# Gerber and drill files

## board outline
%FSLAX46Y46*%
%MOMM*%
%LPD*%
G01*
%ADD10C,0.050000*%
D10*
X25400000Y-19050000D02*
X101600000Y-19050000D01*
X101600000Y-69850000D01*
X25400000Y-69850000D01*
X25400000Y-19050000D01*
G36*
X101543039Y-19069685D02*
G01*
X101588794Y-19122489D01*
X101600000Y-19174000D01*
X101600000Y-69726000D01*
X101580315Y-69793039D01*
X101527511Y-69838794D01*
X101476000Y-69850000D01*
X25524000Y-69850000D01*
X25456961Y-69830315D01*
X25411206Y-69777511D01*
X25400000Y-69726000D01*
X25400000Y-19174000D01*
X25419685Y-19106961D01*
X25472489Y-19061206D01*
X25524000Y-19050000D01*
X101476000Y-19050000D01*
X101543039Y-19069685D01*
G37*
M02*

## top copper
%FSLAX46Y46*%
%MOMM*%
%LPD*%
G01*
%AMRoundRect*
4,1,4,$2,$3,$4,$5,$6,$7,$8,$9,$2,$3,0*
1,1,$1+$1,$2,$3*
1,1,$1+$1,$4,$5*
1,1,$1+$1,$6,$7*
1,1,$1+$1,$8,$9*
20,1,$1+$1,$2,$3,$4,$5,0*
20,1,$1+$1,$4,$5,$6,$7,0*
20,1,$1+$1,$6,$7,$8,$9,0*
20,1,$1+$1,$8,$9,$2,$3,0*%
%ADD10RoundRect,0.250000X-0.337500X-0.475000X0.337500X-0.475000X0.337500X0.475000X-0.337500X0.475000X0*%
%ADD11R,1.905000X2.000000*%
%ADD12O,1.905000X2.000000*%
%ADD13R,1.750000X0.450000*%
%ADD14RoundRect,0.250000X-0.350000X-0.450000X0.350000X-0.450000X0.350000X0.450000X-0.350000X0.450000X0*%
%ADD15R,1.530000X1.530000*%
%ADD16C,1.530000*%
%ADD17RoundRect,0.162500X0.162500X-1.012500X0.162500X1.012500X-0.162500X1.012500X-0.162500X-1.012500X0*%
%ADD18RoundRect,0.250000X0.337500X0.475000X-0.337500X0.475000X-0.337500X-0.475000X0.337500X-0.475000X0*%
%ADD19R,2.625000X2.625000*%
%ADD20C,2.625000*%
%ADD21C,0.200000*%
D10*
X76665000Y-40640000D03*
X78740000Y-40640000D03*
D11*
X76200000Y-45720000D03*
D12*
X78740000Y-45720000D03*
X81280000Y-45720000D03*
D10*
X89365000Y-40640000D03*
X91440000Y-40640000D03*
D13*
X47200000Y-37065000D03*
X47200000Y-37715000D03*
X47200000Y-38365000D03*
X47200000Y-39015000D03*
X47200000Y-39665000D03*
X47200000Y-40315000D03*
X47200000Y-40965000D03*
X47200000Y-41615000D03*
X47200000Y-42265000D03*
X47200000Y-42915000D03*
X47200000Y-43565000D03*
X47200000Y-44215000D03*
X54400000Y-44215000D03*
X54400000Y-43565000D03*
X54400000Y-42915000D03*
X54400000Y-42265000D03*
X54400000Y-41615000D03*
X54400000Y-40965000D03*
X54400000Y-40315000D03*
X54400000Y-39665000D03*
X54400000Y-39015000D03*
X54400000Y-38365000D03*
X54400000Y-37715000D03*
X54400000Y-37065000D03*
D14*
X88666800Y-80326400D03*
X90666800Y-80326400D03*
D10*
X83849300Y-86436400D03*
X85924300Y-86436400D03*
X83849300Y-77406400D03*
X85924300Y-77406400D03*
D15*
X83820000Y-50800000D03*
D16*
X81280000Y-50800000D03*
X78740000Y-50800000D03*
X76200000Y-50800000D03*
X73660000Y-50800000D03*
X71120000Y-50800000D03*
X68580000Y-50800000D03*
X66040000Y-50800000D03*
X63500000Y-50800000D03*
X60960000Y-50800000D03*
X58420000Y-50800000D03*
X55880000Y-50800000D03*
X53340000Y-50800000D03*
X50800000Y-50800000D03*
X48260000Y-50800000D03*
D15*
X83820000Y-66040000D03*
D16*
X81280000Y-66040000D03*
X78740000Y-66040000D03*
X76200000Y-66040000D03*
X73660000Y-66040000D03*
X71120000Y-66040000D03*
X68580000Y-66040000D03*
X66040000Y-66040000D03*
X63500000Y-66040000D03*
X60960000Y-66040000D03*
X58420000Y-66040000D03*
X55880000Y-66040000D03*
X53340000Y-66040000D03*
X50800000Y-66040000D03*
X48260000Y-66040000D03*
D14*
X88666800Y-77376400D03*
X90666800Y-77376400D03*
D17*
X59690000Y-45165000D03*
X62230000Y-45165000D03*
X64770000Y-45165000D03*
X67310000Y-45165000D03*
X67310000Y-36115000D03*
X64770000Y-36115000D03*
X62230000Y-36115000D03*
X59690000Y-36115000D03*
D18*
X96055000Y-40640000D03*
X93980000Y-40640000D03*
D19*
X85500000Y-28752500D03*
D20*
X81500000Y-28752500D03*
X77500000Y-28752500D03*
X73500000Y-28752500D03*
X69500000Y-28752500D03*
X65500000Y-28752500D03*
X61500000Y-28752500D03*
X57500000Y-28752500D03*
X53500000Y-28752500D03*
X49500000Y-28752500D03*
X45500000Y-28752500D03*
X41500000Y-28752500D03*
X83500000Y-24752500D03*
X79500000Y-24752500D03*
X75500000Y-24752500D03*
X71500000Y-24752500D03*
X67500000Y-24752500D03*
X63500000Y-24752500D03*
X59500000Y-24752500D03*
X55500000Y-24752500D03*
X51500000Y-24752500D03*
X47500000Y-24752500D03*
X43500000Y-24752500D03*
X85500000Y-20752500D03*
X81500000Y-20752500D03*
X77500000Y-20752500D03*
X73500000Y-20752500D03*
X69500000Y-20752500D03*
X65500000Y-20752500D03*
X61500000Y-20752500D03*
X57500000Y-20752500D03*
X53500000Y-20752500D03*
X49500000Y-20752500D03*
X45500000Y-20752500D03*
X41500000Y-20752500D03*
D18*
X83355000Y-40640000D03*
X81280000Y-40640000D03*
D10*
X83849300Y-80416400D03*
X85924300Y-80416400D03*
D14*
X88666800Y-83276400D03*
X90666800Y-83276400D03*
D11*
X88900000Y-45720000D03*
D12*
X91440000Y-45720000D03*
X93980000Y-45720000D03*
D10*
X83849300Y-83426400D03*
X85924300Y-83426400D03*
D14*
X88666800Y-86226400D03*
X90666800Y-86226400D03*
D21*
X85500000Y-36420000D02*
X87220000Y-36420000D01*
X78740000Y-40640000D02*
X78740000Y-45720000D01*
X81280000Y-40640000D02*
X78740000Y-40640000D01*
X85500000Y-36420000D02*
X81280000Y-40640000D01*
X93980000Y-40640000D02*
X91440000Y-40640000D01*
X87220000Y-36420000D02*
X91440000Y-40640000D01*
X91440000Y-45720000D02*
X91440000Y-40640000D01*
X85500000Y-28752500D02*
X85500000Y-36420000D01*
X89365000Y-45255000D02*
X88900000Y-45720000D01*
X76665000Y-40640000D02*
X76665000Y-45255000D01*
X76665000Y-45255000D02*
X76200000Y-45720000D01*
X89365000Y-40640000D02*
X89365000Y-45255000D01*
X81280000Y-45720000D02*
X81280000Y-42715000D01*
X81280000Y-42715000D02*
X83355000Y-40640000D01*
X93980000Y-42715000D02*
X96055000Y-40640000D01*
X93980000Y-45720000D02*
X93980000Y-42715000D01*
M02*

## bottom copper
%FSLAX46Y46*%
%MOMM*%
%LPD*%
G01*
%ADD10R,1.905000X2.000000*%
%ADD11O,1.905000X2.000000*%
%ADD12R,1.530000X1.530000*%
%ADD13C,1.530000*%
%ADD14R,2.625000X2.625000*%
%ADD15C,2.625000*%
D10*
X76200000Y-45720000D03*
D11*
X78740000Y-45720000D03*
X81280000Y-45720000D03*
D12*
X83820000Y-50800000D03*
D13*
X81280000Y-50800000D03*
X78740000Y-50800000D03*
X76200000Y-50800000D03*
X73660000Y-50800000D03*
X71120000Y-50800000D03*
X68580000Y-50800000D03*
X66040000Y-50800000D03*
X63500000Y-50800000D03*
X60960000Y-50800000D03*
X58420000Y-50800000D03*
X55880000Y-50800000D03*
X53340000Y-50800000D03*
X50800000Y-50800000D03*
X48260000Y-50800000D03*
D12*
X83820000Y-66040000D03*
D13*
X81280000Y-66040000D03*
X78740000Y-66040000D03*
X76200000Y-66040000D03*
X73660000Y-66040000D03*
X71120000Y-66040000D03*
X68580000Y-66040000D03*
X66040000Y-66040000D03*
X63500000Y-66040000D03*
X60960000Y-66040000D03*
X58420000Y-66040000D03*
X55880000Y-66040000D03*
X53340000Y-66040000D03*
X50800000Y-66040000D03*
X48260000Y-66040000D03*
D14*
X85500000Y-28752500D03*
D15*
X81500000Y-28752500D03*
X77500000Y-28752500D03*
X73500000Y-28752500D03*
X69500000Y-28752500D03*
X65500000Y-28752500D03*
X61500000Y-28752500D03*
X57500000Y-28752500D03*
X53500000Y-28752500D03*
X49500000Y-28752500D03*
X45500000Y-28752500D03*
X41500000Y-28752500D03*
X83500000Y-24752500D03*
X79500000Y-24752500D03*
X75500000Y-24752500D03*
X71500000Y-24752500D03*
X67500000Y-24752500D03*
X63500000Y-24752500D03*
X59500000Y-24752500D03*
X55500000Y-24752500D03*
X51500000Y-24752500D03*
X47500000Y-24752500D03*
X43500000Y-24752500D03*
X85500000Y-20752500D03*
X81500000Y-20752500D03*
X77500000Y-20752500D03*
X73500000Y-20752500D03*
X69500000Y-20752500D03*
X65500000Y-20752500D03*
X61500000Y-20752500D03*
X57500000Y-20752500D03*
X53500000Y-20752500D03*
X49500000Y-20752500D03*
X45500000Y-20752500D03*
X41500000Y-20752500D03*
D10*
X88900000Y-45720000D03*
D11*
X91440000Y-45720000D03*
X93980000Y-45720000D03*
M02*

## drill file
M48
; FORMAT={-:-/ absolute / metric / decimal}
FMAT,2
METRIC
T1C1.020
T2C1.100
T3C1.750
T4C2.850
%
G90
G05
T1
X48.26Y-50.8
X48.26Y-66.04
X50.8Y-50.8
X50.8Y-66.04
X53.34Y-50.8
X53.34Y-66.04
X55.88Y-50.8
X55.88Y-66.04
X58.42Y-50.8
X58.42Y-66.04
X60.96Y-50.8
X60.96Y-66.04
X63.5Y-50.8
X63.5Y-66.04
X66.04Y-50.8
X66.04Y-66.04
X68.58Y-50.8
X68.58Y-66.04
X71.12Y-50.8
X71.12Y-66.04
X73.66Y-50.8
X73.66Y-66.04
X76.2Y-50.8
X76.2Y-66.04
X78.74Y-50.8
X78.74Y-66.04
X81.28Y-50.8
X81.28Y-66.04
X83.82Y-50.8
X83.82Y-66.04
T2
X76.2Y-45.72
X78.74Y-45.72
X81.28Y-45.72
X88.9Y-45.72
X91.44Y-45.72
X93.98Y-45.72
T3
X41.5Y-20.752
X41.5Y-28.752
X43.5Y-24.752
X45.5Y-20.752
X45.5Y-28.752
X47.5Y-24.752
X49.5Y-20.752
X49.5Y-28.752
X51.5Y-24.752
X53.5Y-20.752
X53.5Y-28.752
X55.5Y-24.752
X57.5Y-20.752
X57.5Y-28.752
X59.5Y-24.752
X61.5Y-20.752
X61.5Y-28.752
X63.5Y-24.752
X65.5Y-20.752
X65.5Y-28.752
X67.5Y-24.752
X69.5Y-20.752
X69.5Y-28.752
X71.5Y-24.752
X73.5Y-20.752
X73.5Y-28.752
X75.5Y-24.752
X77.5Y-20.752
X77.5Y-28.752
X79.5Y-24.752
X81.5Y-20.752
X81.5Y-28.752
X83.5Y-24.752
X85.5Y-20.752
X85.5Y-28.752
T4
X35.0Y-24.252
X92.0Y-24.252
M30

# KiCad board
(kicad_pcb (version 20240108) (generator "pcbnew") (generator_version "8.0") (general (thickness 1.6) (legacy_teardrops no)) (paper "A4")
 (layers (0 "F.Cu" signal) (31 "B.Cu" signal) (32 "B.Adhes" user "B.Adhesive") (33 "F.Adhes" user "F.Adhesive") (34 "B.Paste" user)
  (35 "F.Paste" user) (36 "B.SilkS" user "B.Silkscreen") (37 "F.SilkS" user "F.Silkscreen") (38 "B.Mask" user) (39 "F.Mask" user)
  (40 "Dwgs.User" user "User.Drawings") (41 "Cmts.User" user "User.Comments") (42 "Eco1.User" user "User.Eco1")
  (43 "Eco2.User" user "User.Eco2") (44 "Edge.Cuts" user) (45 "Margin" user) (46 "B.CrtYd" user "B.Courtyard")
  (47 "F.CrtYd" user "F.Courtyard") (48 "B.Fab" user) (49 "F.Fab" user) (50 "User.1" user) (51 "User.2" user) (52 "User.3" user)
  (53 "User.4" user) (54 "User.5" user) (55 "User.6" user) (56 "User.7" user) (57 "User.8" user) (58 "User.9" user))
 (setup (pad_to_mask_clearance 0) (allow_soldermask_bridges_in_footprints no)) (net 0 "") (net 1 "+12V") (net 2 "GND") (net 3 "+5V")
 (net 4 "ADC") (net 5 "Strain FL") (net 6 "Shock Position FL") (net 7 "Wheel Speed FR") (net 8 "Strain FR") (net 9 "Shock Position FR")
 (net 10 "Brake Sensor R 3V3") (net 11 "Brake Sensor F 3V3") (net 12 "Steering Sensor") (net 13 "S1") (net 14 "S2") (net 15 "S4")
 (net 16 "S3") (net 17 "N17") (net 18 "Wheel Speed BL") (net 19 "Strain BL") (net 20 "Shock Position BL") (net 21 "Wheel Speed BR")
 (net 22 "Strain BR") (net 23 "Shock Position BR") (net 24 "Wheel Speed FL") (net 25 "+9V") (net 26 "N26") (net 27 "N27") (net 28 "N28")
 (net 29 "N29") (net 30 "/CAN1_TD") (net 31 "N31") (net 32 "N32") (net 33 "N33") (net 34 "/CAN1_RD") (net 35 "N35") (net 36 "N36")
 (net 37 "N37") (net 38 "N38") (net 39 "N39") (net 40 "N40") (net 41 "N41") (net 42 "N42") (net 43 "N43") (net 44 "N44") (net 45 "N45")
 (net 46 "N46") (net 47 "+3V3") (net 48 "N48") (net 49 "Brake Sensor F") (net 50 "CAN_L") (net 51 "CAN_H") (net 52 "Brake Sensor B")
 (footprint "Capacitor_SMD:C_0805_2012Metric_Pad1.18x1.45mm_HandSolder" (layer "F.Cu") (at 77.7025 40.64)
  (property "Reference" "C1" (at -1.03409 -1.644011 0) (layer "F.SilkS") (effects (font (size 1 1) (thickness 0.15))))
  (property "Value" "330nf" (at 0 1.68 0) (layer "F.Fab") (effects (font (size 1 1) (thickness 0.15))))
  (pad "1" smd roundrect (at -1.0375 0) (size 1.175 1.45) (layers "F.Cu" "F.Paste" "F.Mask") (roundrect_rratio 0.212766) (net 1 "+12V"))
  (pad "2" smd roundrect (at 1.0375 0) (size 1.175 1.45) (layers "F.Cu" "F.Paste" "F.Mask") (roundrect_rratio 0.212766) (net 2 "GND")))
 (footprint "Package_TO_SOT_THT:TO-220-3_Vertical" (layer "F.Cu") (at 76.2 45.72)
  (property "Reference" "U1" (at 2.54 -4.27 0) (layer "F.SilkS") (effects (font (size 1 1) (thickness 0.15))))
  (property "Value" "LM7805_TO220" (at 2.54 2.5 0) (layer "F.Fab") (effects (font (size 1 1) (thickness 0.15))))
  (pad "1" thru_hole rect (at 0 0) (size 1.905 2) (drill 1.1) (layers "*.Cu" "*.Mask") (remove_unused_layers no) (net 1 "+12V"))
  (pad "2" thru_hole oval (at 2.54 0) (size 1.905 2) (drill 1.1) (layers "*.Cu" "*.Mask") (remove_unused_layers no) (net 2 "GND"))
  (pad "3" thru_hole oval (at 5.08 0) (size 1.905 2) (drill 1.1) (layers "*.Cu" "*.Mask") (remove_unused_layers no) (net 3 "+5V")))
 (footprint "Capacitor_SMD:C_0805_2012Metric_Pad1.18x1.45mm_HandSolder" (layer "F.Cu") (at 90.4025 40.64)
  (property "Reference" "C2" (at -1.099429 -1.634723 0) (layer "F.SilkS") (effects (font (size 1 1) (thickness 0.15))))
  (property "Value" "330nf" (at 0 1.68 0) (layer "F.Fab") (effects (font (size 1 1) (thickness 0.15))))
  (pad "1" smd roundrect (at -1.0375 0) (size 1.175 1.45) (layers "F.Cu" "F.Paste" "F.Mask") (roundrect_rratio 0.212766) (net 1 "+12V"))
  (pad "2" smd roundrect (at 1.0375 0) (size 1.175 1.45) (layers "F.Cu" "F.Paste" "F.Mask") (roundrect_rratio 0.212766) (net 2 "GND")))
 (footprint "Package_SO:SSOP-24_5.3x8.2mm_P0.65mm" (layer "F.Cu") (at 50.8 40.64)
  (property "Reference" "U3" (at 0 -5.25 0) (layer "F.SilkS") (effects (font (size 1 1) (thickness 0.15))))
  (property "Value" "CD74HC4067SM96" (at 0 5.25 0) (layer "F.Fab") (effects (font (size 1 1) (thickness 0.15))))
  (pad "1" smd rect (at -3.6 -3.575) (size 1.75 0.45) (layers "F.Cu" "F.Paste" "F.Mask") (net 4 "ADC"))
  (pad "2" smd rect (at -3.6 -2.925) (size 1.75 0.45) (layers "F.Cu" "F.Paste" "F.Mask") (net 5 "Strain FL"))
  (pad "3" smd rect (at -3.6 -2.275) (size 1.75 0.45) (layers "F.Cu" "F.Paste" "F.Mask") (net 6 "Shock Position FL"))
  (pad "4" smd rect (at -3.6 -1.625) (size 1.75 0.45) (layers "F.Cu" "F.Paste" "F.Mask") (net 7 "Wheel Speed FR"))
  (pad "5" smd rect (at -3.6 -0.975) (size 1.75 0.45) (layers "F.Cu" "F.Paste" "F.Mask") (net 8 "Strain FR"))
  (pad "6" smd rect (at -3.6 -0.325) (size 1.75 0.45) (layers "F.Cu" "F.Paste" "F.Mask") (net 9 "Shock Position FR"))
  (pad "7" smd rect (at -3.6 0.325) (size 1.75 0.45) (layers "F.Cu" "F.Paste" "F.Mask") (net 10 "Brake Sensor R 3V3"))
  (pad "8" smd rect (at -3.6 0.975) (size 1.75 0.45) (layers "F.Cu" "F.Paste" "F.Mask") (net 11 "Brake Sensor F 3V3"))
  (pad "9" smd rect (at -3.6 1.625) (size 1.75 0.45) (layers "F.Cu" "F.Paste" "F.Mask") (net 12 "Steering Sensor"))
  (pad "10" smd rect (at -3.6 2.275) (size 1.75 0.45) (layers "F.Cu" "F.Paste" "F.Mask") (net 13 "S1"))
  (pad "11" smd rect (at -3.6 2.925) (size 1.75 0.45) (layers "F.Cu" "F.Paste" "F.Mask") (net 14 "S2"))
  (pad "12" smd rect (at -3.6 3.575) (size 1.75 0.45) (layers "F.Cu" "F.Paste" "F.Mask") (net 2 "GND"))
  (pad "13" smd rect (at 3.6 3.575) (size 1.75 0.45) (layers "F.Cu" "F.Paste" "F.Mask") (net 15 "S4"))
  (pad "14" smd rect (at 3.6 2.925) (size 1.75 0.45) (layers "F.Cu" "F.Paste" "F.Mask") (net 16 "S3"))
  (pad "15" smd rect (at 3.6 2.275) (size 1.75 0.45) (layers "F.Cu" "F.Paste" "F.Mask") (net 2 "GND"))
  (pad "16" smd rect (at 3.6 1.625) (size 1.75 0.45) (layers "F.Cu" "F.Paste" "F.Mask") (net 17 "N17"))
  (pad "17" smd rect (at 3.6 0.975) (size 1.75 0.45) (layers "F.Cu" "F.Paste" "F.Mask") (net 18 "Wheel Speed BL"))
  (pad "18" smd rect (at 3.6 0.325) (size 1.75 0.45) (layers "F.Cu" "F.Paste" "F.Mask") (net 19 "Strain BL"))
  (pad "19" smd rect (at 3.6 -0.325) (size 1.75 0.45) (layers "F.Cu" "F.Paste" "F.Mask") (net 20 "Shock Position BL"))
  (pad "20" smd rect (at 3.6 -0.975) (size 1.75 0.45) (layers "F.Cu" "F.Paste" "F.Mask") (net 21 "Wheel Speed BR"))
  (pad "21" smd rect (at 3.6 -1.625) (size 1.75 0.45) (layers "F.Cu" "F.Paste" "F.Mask") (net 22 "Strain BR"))
  (pad "22" smd rect (at 3.6 -2.275) (size 1.75 0.45) (layers "F.Cu" "F.Paste" "F.Mask") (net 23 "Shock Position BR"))
  (pad "23" smd rect (at 3.6 -2.925) (size 1.75 0.45) (layers "F.Cu" "F.Paste" "F.Mask") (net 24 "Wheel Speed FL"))
  (pad "24" smd rect (at 3.6 -3.575) (size 1.75 0.45) (layers "F.Cu" "F.Paste" "F.Mask") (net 3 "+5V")))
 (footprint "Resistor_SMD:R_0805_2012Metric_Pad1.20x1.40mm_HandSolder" (layer "F.Cu") (at 89.6668 80.3264)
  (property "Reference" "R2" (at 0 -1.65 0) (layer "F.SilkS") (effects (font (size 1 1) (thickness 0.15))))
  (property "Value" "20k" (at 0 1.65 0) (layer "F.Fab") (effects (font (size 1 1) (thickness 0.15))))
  (pad "1" smd roundrect (at -1 0) (size 1.2 1.4) (layers "F.Cu" "F.Paste" "F.Mask") (roundrect_rratio 0.208333) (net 2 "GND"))
  (pad "2" smd roundrect (at 1 0) (size 1.2 1.4) (layers "F.Cu" "F.Paste" "F.Mask") (roundrect_rratio 0.208333)
   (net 11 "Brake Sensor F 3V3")))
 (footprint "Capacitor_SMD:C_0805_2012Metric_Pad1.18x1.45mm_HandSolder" (layer "F.Cu") (at 84.8868 86.4364)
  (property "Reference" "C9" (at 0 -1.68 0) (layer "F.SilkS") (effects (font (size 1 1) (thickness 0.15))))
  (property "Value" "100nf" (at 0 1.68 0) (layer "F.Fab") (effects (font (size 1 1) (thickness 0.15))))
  (pad "1" smd roundrect (at -1.0375 0) (size 1.175 1.45) (layers "F.Cu" "F.Paste" "F.Mask") (roundrect_rratio 0.212766) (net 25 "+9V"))
  (pad "2" smd roundrect (at 1.0375 0) (size 1.175 1.45) (layers "F.Cu" "F.Paste" "F.Mask") (roundrect_rratio 0.212766) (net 2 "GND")))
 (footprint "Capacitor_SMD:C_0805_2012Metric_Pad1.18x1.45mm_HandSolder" (layer "F.Cu") (at 84.8868 77.4064)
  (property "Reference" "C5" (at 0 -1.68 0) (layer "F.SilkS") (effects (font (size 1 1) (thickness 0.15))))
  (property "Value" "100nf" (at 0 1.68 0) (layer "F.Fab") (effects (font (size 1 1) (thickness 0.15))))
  (pad "1" smd roundrect (at -1.0375 0) (size 1.175 1.45) (layers "F.Cu" "F.Paste" "F.Mask") (roundrect_rratio 0.212766) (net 3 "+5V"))
  (pad "2" smd roundrect (at 1.0375 0) (size 1.175 1.45) (layers "F.Cu" "F.Paste" "F.Mask") (roundrect_rratio 0.212766) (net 2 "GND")))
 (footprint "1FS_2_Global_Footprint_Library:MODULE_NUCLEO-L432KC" (layer "F.Cu") (at 67.605 58.42 -90)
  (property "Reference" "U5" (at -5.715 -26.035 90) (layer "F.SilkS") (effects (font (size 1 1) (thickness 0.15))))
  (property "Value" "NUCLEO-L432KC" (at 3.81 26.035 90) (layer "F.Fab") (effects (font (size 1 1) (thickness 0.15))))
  (pad "CN3_1" thru_hole rect (at -7.62 -16.215 270) (size 1.53 1.53) (drill 1.02) (layers "*.Cu" "*.Mask") (remove_unused_layers no)
   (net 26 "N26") (solder_mask_margin 0.102))
  (pad "CN3_2" thru_hole circle (at -7.62 -13.675 270) (size 1.53 1.53) (drill 1.02) (layers "*.Cu" "*.Mask") (remove_unused_layers no)
   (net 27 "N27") (solder_mask_margin 0.102))
  (pad "CN3_3" thru_hole circle (at -7.62 -11.135 270) (size 1.53 1.53) (drill 1.02) (layers "*.Cu" "*.Mask") (remove_unused_layers no)
   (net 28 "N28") (solder_mask_margin 0.102))
  (pad "CN3_4" thru_hole circle (at -7.62 -8.595 270) (size 1.53 1.53) (drill 1.02) (layers "*.Cu" "*.Mask") (remove_unused_layers no)
   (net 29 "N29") (solder_mask_margin 0.102))
  (pad "CN3_5" thru_hole circle (at -7.62 -6.055 270) (size 1.53 1.53) (drill 1.02) (layers "*.Cu" "*.Mask") (remove_unused_layers no)
   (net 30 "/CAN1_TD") (solder_mask_margin 0.102))
  (pad "CN3_6" thru_hole circle (at -7.62 -3.515 270) (size 1.53 1.53) (drill 1.02) (layers "*.Cu" "*.Mask") (remove_unused_layers no)
   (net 13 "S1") (solder_mask_margin 0.102))
  (pad "CN3_7" thru_hole circle (at -7.62 -0.975 270) (size 1.53 1.53) (drill 1.02) (layers "*.Cu" "*.Mask") (remove_unused_layers no)
   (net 14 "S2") (solder_mask_margin 0.102))
  (pad "CN3_8" thru_hole circle (at -7.62 1.565 270) (size 1.53 1.53) (drill 1.02) (layers "*.Cu" "*.Mask") (remove_unused_layers no)
   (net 16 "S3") (solder_mask_margin 0.102))
  (pad "CN3_9" thru_hole circle (at -7.62 4.105 270) (size 1.53 1.53) (drill 1.02) (layers "*.Cu" "*.Mask") (remove_unused_layers no)
   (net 15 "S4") (solder_mask_margin 0.102))
  (pad "CN3_10" thru_hole circle (at -7.62 6.645 270) (size 1.53 1.53) (drill 1.02) (layers "*.Cu" "*.Mask") (remove_unused_layers no)
   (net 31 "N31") (solder_mask_margin 0.102))
  (pad "CN3_11" thru_hole circle (at -7.62 9.185 270) (size 1.53 1.53) (drill 1.02) (layers "*.Cu" "*.Mask") (remove_unused_layers no)
   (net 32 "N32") (solder_mask_margin 0.102))
  (pad "CN3_12" thru_hole circle (at -7.62 11.725 270) (size 1.53 1.53) (drill 1.02) (layers "*.Cu" "*.Mask") (remove_unused_layers no)
   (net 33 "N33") (solder_mask_margin 0.102))
  (pad "CN3_13" thru_hole circle (at -7.62 14.265 270) (size 1.53 1.53) (drill 1.02) (layers "*.Cu" "*.Mask") (remove_unused_layers no)
   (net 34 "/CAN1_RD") (solder_mask_margin 0.102))
  (pad "CN3_14" thru_hole circle (at -7.62 16.805 270) (size 1.53 1.53) (drill 1.02) (layers "*.Cu" "*.Mask") (remove_unused_layers no)
   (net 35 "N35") (solder_mask_margin 0.102))
  (pad "CN3_15" thru_hole circle (at -7.62 19.345 270) (size 1.53 1.53) (drill 1.02) (layers "*.Cu" "*.Mask") (remove_unused_layers no)
   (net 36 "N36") (solder_mask_margin 0.102))
  (pad "CN4_1" thru_hole rect (at 7.62 -16.215 270) (size 1.53 1.53) (drill 1.02) (layers "*.Cu" "*.Mask") (remove_unused_layers no)
   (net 25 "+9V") (solder_mask_margin 0.102))
  (pad "CN4_2" thru_hole circle (at 7.62 -13.675 270) (size 1.53 1.53) (drill 1.02) (layers "*.Cu" "*.Mask") (remove_unused_layers no)
   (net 2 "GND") (solder_mask_margin 0.102))
  (pad "CN4_3" thru_hole circle (at 7.62 -11.135 270) (size 1.53 1.53) (drill 1.02) (layers "*.Cu" "*.Mask") (remove_unused_layers no)
   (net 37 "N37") (solder_mask_margin 0.102))
  (pad "CN4_4" thru_hole circle (at 7.62 -8.595 270) (size 1.53 1.53) (drill 1.02) (layers "*.Cu" "*.Mask") (remove_unused_layers no)
   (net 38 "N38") (solder_mask_margin 0.102))
  (pad "CN4_5" thru_hole circle (at 7.62 -6.055 270) (size 1.53 1.53) (drill 1.02) (layers "*.Cu" "*.Mask") (remove_unused_layers no)
   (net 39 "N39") (solder_mask_margin 0.102))
  (pad "CN4_6" thru_hole circle (at 7.62 -3.515 270) (size 1.53 1.53) (drill 1.02) (layers "*.Cu" "*.Mask") (remove_unused_layers no)
   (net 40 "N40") (solder_mask_margin 0.102))
  (pad "CN4_7" thru_hole circle (at 7.62 -0.975 270) (size 1.53 1.53) (drill 1.02) (layers "*.Cu" "*.Mask") (remove_unused_layers no)
   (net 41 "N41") (solder_mask_margin 0.102))
  (pad "CN4_8" thru_hole circle (at 7.62 1.565 270) (size 1.53 1.53) (drill 1.02) (layers "*.Cu" "*.Mask") (remove_unused_layers no)
   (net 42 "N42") (solder_mask_margin 0.102))
  (pad "CN4_9" thru_hole circle (at 7.62 4.105 270) (size 1.53 1.53) (drill 1.02) (layers "*.Cu" "*.Mask") (remove_unused_layers no)
   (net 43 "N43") (solder_mask_margin 0.102))
  (pad "CN4_10" thru_hole circle (at 7.62 6.645 270) (size 1.53 1.53) (drill 1.02) (layers "*.Cu" "*.Mask") (remove_unused_layers no)
   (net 4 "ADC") (solder_mask_margin 0.102))
  (pad "CN4_11" thru_hole circle (at 7.62 9.185 270) (size 1.53 1.53) (drill 1.02) (layers "*.Cu" "*.Mask") (remove_unused_layers no)
   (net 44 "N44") (solder_mask_margin 0.102))
  (pad "CN4_12" thru_hole circle (at 7.62 11.725 270) (size 1.53 1.53) (drill 1.02) (layers "*.Cu" "*.Mask") (remove_unused_layers no)
   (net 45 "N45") (solder_mask_margin 0.102))
  (pad "CN4_13" thru_hole circle (at 7.62 14.265 270) (size 1.53 1.53) (drill 1.02) (layers "*.Cu" "*.Mask") (remove_unused_layers no)
   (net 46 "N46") (solder_mask_margin 0.102))
  (pad "CN4_14" thru_hole circle (at 7.62 16.805 270) (size 1.53 1.53) (drill 1.02) (layers "*.Cu" "*.Mask") (remove_unused_layers no)
   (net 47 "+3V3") (solder_mask_margin 0.102))
  (pad "CN4_15" thru_hole circle (at 7.62 19.345 270) (size 1.53 1.53) (drill 1.02) (layers "*.Cu" "*.Mask") (remove_unused_layers no)
   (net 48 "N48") (solder_mask_margin 0.102)))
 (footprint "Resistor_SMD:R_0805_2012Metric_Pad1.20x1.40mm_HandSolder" (layer "F.Cu") (at 89.6668 77.3764)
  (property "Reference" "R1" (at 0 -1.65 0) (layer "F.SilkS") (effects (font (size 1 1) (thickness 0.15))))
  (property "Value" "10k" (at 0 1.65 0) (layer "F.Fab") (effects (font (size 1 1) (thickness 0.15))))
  (pad "1" smd roundrect (at -1 0) (size 1.2 1.4) (layers "F.Cu" "F.Paste" "F.Mask") (roundrect_rratio 0.208333) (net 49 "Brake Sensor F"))
  (pad "2" smd roundrect (at 1 0) (size 1.2 1.4) (layers "F.Cu" "F.Paste" "F.Mask") (roundrect_rratio 0.208333)
   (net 11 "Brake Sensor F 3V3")))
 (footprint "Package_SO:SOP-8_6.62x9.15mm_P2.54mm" (layer "F.Cu") (at 63.5 40.64 90)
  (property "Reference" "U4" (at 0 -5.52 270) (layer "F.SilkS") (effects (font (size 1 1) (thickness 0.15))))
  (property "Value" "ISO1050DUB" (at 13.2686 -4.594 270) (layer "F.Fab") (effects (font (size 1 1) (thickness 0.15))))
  (pad "1" smd roundrect (at -4.525 -3.81 90) (size 2.35 0.65) (layers "F.Cu" "F.Paste" "F.Mask") (roundrect_rratio 0.25) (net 47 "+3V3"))
  (pad "2" smd roundrect (at -4.525 -1.27 90) (size 2.35 0.65) (layers "F.Cu" "F.Paste" "F.Mask") (roundrect_rratio 0.25)
   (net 34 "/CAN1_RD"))
  (pad "3" smd roundrect (at -4.525 1.27 90) (size 2.35 0.65) (layers "F.Cu" "F.Paste" "F.Mask") (roundrect_rratio 0.25) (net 30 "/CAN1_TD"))
  (pad "4" smd roundrect (at -4.525 3.81 90) (size 2.35 0.65) (layers "F.Cu" "F.Paste" "F.Mask") (roundrect_rratio 0.25) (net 2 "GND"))
  (pad "5" smd roundrect (at 4.525 3.81 90) (size 2.35 0.65) (layers "F.Cu" "F.Paste" "F.Mask") (roundrect_rratio 0.25) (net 2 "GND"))
  (pad "6" smd roundrect (at 4.525 1.27 90) (size 2.35 0.65) (layers "F.Cu" "F.Paste" "F.Mask") (roundrect_rratio 0.25) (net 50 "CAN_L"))
  (pad "7" smd roundrect (at 4.525 -1.27 90) (size 2.35 0.65) (layers "F.Cu" "F.Paste" "F.Mask") (roundrect_rratio 0.25) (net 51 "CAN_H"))
  (pad "8" smd roundrect (at 4.525 -3.81 90) (size 2.35 0.65) (layers "F.Cu" "F.Paste" "F.Mask") (roundrect_rratio 0.25) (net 3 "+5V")))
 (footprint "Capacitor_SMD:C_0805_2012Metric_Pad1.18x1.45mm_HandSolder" (layer "F.Cu") (at 95.0175 40.64 180)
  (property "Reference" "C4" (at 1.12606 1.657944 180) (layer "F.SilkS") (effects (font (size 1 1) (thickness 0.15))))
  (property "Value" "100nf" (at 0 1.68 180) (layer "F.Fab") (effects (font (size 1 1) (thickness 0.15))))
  (pad "1" smd roundrect (at -1.0375 0 180) (size 1.175 1.45) (layers "F.Cu" "F.Paste" "F.Mask") (roundrect_rratio 0.212766) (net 25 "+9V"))
  (pad "2" smd roundrect (at 1.0375 0 180) (size 1.175 1.45) (layers "F.Cu" "F.Paste" "F.Mask") (roundrect_rratio 0.212766) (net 2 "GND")))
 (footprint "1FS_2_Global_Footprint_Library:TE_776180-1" (layer "F.Cu") (at 63.5 24.7525 180)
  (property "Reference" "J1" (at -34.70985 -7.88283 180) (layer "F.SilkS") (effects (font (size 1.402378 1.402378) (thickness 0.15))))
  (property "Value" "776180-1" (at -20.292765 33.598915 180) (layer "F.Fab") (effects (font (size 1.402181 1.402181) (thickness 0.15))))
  (pad "" np_thru_hole circle (at -28.5 0.5 180) (size 2.85 2.85) (drill 2.85) (layers "*.Cu" "*.Mask"))
  (pad "" np_thru_hole circle (at 28.5 0.5 180) (size 2.85 2.85) (drill 2.85) (layers "*.Cu" "*.Mask"))
  (pad "1" thru_hole rect (at -22 -4 180) (size 2.625 2.625) (drill 1.75) (layers "*.Cu" "*.Mask") (remove_unused_layers no) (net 2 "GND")
   (solder_mask_margin 0.102))
  (pad "2" thru_hole circle (at -18 -4 180) (size 2.625 2.625) (drill 1.75) (layers "*.Cu" "*.Mask") (remove_unused_layers no) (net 3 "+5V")
   (solder_mask_margin 0.102))
  (pad "3" thru_hole circle (at -14 -4 180) (size 2.625 2.625) (drill 1.75) (layers "*.Cu" "*.Mask") (remove_unused_layers no)
   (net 47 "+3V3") (solder_mask_margin 0.102))
  (pad "4" thru_hole circle (at -10 -4 180) (size 2.625 2.625) (drill 1.75) (layers "*.Cu" "*.Mask") (remove_unused_layers no)
   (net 9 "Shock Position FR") (solder_mask_margin 0.102))
  (pad "5" thru_hole circle (at -6 -4 180) (size 2.625 2.625) (drill 1.75) (layers "*.Cu" "*.Mask") (remove_unused_layers no)
   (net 8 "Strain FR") (solder_mask_margin 0.102))
  (pad "6" thru_hole circle (at -2 -4 180) (size 2.625 2.625) (drill 1.75) (layers "*.Cu" "*.Mask") (remove_unused_layers no)
   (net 7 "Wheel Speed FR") (solder_mask_margin 0.102))
  (pad "7" thru_hole circle (at 2 -4 180) (size 2.625 2.625) (drill 1.75) (layers "*.Cu" "*.Mask") (remove_unused_layers no) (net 2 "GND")
   (solder_mask_margin 0.102))
  (pad "8" thru_hole circle (at 6 -4 180) (size 2.625 2.625) (drill 1.75) (layers "*.Cu" "*.Mask") (remove_unused_layers no) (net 3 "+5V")
   (solder_mask_margin 0.102))
  (pad "9" thru_hole circle (at 10 -4 180) (size 2.625 2.625) (drill 1.75) (layers "*.Cu" "*.Mask") (remove_unused_layers no)
   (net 47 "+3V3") (solder_mask_margin 0.102))
  (pad "10" thru_hole circle (at 14 -4 180) (size 2.625 2.625) (drill 1.75) (layers "*.Cu" "*.Mask") (remove_unused_layers no)
   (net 6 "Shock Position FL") (solder_mask_margin 0.102))
  (pad "11" thru_hole circle (at 18 -4 180) (size 2.625 2.625) (drill 1.75) (layers "*.Cu" "*.Mask") (remove_unused_layers no)
   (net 5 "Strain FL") (solder_mask_margin 0.102))
  (pad "12" thru_hole circle (at 22 -4 180) (size 2.625 2.625) (drill 1.75) (layers "*.Cu" "*.Mask") (remove_unused_layers no)
   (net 24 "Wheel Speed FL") (solder_mask_margin 0.102))
  (pad "13" thru_hole circle (at -20 0 180) (size 2.625 2.625) (drill 1.75) (layers "*.Cu" "*.Mask") (remove_unused_layers no) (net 2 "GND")
   (solder_mask_margin 0.102))
  (pad "14" thru_hole circle (at -16 0 180) (size 2.625 2.625) (drill 1.75) (layers "*.Cu" "*.Mask") (remove_unused_layers no)
   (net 1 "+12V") (solder_mask_margin 0.102))
  (pad "15" thru_hole circle (at -12 0 180) (size 2.625 2.625) (drill 1.75) (layers "*.Cu" "*.Mask") (remove_unused_layers no)
   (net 51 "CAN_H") (solder_mask_margin 0.102))
  (pad "16" thru_hole circle (at -8 0 180) (size 2.625 2.625) (drill 1.75) (layers "*.Cu" "*.Mask") (remove_unused_layers no)
   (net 50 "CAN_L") (solder_mask_margin 0.102))
  (pad "17" thru_hole circle (at -4 0 180) (size 2.625 2.625) (drill 1.75) (layers "*.Cu" "*.Mask") (remove_unused_layers no)
   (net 51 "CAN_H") (solder_mask_margin 0.102))
  (pad "18" thru_hole circle (at 0 0 180) (size 2.625 2.625) (drill 1.75) (layers "*.Cu" "*.Mask") (remove_unused_layers no)
   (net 50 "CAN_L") (solder_mask_margin 0.102))
  (pad "19" thru_hole circle (at 4 0 180) (size 2.625 2.625) (drill 1.75) (layers "*.Cu" "*.Mask") (remove_unused_layers no) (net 2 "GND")
   (solder_mask_margin 0.102))
  (pad "20" thru_hole circle (at 8 0 180) (size 2.625 2.625) (drill 1.75) (layers "*.Cu" "*.Mask") (remove_unused_layers no) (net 47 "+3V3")
   (solder_mask_margin 0.102))
  (pad "21" thru_hole circle (at 12 0 180) (size 2.625 2.625) (drill 1.75) (layers "*.Cu" "*.Mask") (remove_unused_layers no)
   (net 12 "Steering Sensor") (solder_mask_margin 0.102))
  (pad "22" thru_hole circle (at 16 0 180) (size 2.625 2.625) (drill 1.75) (layers "*.Cu" "*.Mask") (remove_unused_layers no)
   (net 49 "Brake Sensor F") (solder_mask_margin 0.102))
  (pad "23" thru_hole circle (at 20 0 180) (size 2.625 2.625) (drill 1.75) (layers "*.Cu" "*.Mask") (remove_unused_layers no)
   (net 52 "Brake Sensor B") (solder_mask_margin 0.102))
  (pad "24" thru_hole circle (at -22 4 180) (size 2.625 2.625) (drill 1.75) (layers "*.Cu" "*.Mask") (remove_unused_layers no) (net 2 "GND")
   (solder_mask_margin 0.102))
  (pad "25" thru_hole circle (at -18 4 180) (size 2.625 2.625) (drill 1.75) (layers "*.Cu" "*.Mask") (remove_unused_layers no) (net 3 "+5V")
   (solder_mask_margin 0.102))
  (pad "26" thru_hole circle (at -14 4 180) (size 2.625 2.625) (drill 1.75) (layers "*.Cu" "*.Mask") (remove_unused_layers no)
   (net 47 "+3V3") (solder_mask_margin 0.102))
  (pad "27" thru_hole circle (at -10 4 180) (size 2.625 2.625) (drill 1.75) (layers "*.Cu" "*.Mask") (remove_unused_layers no)
   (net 23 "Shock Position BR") (solder_mask_margin 0.102))
  (pad "28" thru_hole circle (at -6 4 180) (size 2.625 2.625) (drill 1.75) (layers "*.Cu" "*.Mask") (remove_unused_layers no)
   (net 22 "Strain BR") (solder_mask_margin 0.102))
  (pad "29" thru_hole circle (at -2 4 180) (size 2.625 2.625) (drill 1.75) (layers "*.Cu" "*.Mask") (remove_unused_layers no)
   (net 21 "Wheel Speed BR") (solder_mask_margin 0.102))
  (pad "30" thru_hole circle (at 2 4 180) (size 2.625 2.625) (drill 1.75) (layers "*.Cu" "*.Mask") (remove_unused_layers no) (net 2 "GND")
   (solder_mask_margin 0.102))
  (pad "31" thru_hole circle (at 6 4 180) (size 2.625 2.625) (drill 1.75) (layers "*.Cu" "*.Mask") (remove_unused_layers no) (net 3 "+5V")
   (solder_mask_margin 0.102))
  (pad "32" thru_hole circle (at 10 4 180) (size 2.625 2.625) (drill 1.75) (layers "*.Cu" "*.Mask") (remove_unused_layers no)
   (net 47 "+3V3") (solder_mask_margin 0.102))
  (pad "33" thru_hole circle (at 14 4 180) (size 2.625 2.625) (drill 1.75) (layers "*.Cu" "*.Mask") (remove_unused_layers no)
   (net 20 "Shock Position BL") (solder_mask_margin 0.102))
  (pad "34" thru_hole circle (at 18 4 180) (size 2.625 2.625) (drill 1.75) (layers "*.Cu" "*.Mask") (remove_unused_layers no)
   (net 19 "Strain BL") (solder_mask_margin 0.102))
  (pad "35" thru_hole circle (at 22 4 180) (size 2.625 2.625) (drill 1.75) (layers "*.Cu" "*.Mask") (remove_unused_layers no)
   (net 18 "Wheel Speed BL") (solder_mask_margin 0.102)))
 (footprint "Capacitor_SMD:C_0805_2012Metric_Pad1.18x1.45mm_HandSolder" (layer "F.Cu") (at 82.3175 40.64 180)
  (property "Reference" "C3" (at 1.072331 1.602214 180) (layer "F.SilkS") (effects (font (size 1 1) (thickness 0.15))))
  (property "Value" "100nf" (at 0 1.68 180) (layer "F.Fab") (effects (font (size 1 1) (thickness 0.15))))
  (pad "1" smd roundrect (at -1.0375 0 180) (size 1.175 1.45) (layers "F.Cu" "F.Paste" "F.Mask") (roundrect_rratio 0.212766) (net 3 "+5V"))
  (pad "2" smd roundrect (at 1.0375 0 180) (size 1.175 1.45) (layers "F.Cu" "F.Paste" "F.Mask") (roundrect_rratio 0.212766) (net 2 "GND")))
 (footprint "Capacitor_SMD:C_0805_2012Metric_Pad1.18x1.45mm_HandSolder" (layer "F.Cu") (at 84.8868 80.4164)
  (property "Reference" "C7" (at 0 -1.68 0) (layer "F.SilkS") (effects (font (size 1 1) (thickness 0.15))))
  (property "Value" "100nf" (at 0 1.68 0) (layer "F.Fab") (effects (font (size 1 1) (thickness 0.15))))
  (pad "1" smd roundrect (at -1.0375 0) (size 1.175 1.45) (layers "F.Cu" "F.Paste" "F.Mask") (roundrect_rratio 0.212766) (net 2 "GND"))
  (pad "2" smd roundrect (at 1.0375 0) (size 1.175 1.45) (layers "F.Cu" "F.Paste" "F.Mask") (roundrect_rratio 0.212766) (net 3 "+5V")))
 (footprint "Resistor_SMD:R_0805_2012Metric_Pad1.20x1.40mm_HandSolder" (layer "F.Cu") (at 89.6668 83.2764)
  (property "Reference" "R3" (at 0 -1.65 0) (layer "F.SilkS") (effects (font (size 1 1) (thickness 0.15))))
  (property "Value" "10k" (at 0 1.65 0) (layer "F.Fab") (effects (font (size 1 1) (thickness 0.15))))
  (pad "1" smd roundrect (at -1 0) (size 1.2 1.4) (layers "F.Cu" "F.Paste" "F.Mask") (roundrect_rratio 0.208333) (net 52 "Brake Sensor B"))
  (pad "2" smd roundrect (at 1 0) (size 1.2 1.4) (layers "F.Cu" "F.Paste" "F.Mask") (roundrect_rratio 0.208333)
   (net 10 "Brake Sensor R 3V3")))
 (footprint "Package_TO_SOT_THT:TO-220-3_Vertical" (layer "F.Cu") (at 88.9 45.72)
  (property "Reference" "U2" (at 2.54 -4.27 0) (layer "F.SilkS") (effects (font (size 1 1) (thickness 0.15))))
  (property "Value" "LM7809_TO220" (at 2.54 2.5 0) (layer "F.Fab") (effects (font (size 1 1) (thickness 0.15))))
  (pad "1" thru_hole rect (at 0 0) (size 1.905 2) (drill 1.1) (layers "*.Cu" "*.Mask") (remove_unused_layers no) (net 1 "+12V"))
  (pad "2" thru_hole oval (at 2.54 0) (size 1.905 2) (drill 1.1) (layers "*.Cu" "*.Mask") (remove_unused_layers no) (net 2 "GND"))
  (pad "3" thru_hole oval (at 5.08 0) (size 1.905 2) (drill 1.1) (layers "*.Cu" "*.Mask") (remove_unused_layers no) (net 25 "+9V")))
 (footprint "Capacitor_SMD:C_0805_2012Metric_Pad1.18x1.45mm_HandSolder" (layer "F.Cu") (at 84.8868 83.4264)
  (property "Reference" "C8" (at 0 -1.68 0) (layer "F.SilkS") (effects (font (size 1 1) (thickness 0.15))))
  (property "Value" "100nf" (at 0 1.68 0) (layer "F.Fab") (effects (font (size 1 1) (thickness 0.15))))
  (pad "1" smd roundrect (at -1.0375 0) (size 1.175 1.45) (layers "F.Cu" "F.Paste" "F.Mask") (roundrect_rratio 0.212766) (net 2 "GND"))
  (pad "2" smd roundrect (at 1.0375 0) (size 1.175 1.45) (layers "F.Cu" "F.Paste" "F.Mask") (roundrect_rratio 0.212766) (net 47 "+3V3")))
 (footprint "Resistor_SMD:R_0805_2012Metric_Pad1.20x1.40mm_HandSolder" (layer "F.Cu") (at 89.6668 86.2264)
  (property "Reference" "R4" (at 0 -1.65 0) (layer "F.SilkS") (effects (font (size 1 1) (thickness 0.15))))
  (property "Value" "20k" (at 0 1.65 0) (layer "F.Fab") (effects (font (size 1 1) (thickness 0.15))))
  (pad "1" smd roundrect (at -1 0) (size 1.2 1.4) (layers "F.Cu" "F.Paste" "F.Mask") (roundrect_rratio 0.208333) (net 2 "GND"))
  (pad "2" smd roundrect (at 1 0) (size 1.2 1.4) (layers "F.Cu" "F.Paste" "F.Mask") (roundrect_rratio 0.208333)
   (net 10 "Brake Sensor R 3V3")))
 (gr_rect (start 25.4 19.05) (end 101.6 69.85) (stroke (width 0.05) (type default)) (fill none) (layer "Edge.Cuts"))
 (segment (start 85.5 36.42) (end 87.22 36.42) (width 0.2) (layer "F.Cu") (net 2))
 (segment (start 78.74 40.64) (end 78.74 45.72) (width 0.2) (layer "F.Cu") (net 2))
 (segment (start 81.28 40.64) (end 78.74 40.64) (width 0.2) (layer "F.Cu") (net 2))
 (segment (start 85.5 36.42) (end 81.28 40.64) (width 0.2) (layer "F.Cu") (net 2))
 (segment (start 93.98 40.64) (end 91.44 40.64) (width 0.2) (layer "F.Cu") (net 2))
 (segment (start 87.22 36.42) (end 91.44 40.64) (width 0.2) (layer "F.Cu") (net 2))
 (segment (start 91.44 45.72) (end 91.44 40.64) (width 0.2) (layer "F.Cu") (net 2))
 (segment (start 85.5 28.7525) (end 85.5 36.42) (width 0.2) (layer "F.Cu") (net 2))
 (segment (start 89.365 45.255) (end 88.9 45.72) (width 0.2) (layer "F.Cu") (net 1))
 (segment (start 76.665 40.64) (end 76.665 45.255) (width 0.2) (layer "F.Cu") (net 1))
 (segment (start 76.665 45.255) (end 76.2 45.72) (width 0.2) (layer "F.Cu") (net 1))
 (segment (start 89.365 40.64) (end 89.365 45.255) (width 0.2) (layer "F.Cu") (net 1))
 (segment (start 81.28 45.72) (end 81.28 42.715) (width 0.2) (layer "F.Cu") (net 3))
 (segment (start 81.28 42.715) (end 83.355 40.64) (width 0.2) (layer "F.Cu") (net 3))
 (segment (start 93.98 42.715) (end 96.055 40.64) (width 0.2) (layer "F.Cu") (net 25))
 (segment (start 93.98 45.72) (end 93.98 42.715) (width 0.2) (layer "F.Cu") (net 25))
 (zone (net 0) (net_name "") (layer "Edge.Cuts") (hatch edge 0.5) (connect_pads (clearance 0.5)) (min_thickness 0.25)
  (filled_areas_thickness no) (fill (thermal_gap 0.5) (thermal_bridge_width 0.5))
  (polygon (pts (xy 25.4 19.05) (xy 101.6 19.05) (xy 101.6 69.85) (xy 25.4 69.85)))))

